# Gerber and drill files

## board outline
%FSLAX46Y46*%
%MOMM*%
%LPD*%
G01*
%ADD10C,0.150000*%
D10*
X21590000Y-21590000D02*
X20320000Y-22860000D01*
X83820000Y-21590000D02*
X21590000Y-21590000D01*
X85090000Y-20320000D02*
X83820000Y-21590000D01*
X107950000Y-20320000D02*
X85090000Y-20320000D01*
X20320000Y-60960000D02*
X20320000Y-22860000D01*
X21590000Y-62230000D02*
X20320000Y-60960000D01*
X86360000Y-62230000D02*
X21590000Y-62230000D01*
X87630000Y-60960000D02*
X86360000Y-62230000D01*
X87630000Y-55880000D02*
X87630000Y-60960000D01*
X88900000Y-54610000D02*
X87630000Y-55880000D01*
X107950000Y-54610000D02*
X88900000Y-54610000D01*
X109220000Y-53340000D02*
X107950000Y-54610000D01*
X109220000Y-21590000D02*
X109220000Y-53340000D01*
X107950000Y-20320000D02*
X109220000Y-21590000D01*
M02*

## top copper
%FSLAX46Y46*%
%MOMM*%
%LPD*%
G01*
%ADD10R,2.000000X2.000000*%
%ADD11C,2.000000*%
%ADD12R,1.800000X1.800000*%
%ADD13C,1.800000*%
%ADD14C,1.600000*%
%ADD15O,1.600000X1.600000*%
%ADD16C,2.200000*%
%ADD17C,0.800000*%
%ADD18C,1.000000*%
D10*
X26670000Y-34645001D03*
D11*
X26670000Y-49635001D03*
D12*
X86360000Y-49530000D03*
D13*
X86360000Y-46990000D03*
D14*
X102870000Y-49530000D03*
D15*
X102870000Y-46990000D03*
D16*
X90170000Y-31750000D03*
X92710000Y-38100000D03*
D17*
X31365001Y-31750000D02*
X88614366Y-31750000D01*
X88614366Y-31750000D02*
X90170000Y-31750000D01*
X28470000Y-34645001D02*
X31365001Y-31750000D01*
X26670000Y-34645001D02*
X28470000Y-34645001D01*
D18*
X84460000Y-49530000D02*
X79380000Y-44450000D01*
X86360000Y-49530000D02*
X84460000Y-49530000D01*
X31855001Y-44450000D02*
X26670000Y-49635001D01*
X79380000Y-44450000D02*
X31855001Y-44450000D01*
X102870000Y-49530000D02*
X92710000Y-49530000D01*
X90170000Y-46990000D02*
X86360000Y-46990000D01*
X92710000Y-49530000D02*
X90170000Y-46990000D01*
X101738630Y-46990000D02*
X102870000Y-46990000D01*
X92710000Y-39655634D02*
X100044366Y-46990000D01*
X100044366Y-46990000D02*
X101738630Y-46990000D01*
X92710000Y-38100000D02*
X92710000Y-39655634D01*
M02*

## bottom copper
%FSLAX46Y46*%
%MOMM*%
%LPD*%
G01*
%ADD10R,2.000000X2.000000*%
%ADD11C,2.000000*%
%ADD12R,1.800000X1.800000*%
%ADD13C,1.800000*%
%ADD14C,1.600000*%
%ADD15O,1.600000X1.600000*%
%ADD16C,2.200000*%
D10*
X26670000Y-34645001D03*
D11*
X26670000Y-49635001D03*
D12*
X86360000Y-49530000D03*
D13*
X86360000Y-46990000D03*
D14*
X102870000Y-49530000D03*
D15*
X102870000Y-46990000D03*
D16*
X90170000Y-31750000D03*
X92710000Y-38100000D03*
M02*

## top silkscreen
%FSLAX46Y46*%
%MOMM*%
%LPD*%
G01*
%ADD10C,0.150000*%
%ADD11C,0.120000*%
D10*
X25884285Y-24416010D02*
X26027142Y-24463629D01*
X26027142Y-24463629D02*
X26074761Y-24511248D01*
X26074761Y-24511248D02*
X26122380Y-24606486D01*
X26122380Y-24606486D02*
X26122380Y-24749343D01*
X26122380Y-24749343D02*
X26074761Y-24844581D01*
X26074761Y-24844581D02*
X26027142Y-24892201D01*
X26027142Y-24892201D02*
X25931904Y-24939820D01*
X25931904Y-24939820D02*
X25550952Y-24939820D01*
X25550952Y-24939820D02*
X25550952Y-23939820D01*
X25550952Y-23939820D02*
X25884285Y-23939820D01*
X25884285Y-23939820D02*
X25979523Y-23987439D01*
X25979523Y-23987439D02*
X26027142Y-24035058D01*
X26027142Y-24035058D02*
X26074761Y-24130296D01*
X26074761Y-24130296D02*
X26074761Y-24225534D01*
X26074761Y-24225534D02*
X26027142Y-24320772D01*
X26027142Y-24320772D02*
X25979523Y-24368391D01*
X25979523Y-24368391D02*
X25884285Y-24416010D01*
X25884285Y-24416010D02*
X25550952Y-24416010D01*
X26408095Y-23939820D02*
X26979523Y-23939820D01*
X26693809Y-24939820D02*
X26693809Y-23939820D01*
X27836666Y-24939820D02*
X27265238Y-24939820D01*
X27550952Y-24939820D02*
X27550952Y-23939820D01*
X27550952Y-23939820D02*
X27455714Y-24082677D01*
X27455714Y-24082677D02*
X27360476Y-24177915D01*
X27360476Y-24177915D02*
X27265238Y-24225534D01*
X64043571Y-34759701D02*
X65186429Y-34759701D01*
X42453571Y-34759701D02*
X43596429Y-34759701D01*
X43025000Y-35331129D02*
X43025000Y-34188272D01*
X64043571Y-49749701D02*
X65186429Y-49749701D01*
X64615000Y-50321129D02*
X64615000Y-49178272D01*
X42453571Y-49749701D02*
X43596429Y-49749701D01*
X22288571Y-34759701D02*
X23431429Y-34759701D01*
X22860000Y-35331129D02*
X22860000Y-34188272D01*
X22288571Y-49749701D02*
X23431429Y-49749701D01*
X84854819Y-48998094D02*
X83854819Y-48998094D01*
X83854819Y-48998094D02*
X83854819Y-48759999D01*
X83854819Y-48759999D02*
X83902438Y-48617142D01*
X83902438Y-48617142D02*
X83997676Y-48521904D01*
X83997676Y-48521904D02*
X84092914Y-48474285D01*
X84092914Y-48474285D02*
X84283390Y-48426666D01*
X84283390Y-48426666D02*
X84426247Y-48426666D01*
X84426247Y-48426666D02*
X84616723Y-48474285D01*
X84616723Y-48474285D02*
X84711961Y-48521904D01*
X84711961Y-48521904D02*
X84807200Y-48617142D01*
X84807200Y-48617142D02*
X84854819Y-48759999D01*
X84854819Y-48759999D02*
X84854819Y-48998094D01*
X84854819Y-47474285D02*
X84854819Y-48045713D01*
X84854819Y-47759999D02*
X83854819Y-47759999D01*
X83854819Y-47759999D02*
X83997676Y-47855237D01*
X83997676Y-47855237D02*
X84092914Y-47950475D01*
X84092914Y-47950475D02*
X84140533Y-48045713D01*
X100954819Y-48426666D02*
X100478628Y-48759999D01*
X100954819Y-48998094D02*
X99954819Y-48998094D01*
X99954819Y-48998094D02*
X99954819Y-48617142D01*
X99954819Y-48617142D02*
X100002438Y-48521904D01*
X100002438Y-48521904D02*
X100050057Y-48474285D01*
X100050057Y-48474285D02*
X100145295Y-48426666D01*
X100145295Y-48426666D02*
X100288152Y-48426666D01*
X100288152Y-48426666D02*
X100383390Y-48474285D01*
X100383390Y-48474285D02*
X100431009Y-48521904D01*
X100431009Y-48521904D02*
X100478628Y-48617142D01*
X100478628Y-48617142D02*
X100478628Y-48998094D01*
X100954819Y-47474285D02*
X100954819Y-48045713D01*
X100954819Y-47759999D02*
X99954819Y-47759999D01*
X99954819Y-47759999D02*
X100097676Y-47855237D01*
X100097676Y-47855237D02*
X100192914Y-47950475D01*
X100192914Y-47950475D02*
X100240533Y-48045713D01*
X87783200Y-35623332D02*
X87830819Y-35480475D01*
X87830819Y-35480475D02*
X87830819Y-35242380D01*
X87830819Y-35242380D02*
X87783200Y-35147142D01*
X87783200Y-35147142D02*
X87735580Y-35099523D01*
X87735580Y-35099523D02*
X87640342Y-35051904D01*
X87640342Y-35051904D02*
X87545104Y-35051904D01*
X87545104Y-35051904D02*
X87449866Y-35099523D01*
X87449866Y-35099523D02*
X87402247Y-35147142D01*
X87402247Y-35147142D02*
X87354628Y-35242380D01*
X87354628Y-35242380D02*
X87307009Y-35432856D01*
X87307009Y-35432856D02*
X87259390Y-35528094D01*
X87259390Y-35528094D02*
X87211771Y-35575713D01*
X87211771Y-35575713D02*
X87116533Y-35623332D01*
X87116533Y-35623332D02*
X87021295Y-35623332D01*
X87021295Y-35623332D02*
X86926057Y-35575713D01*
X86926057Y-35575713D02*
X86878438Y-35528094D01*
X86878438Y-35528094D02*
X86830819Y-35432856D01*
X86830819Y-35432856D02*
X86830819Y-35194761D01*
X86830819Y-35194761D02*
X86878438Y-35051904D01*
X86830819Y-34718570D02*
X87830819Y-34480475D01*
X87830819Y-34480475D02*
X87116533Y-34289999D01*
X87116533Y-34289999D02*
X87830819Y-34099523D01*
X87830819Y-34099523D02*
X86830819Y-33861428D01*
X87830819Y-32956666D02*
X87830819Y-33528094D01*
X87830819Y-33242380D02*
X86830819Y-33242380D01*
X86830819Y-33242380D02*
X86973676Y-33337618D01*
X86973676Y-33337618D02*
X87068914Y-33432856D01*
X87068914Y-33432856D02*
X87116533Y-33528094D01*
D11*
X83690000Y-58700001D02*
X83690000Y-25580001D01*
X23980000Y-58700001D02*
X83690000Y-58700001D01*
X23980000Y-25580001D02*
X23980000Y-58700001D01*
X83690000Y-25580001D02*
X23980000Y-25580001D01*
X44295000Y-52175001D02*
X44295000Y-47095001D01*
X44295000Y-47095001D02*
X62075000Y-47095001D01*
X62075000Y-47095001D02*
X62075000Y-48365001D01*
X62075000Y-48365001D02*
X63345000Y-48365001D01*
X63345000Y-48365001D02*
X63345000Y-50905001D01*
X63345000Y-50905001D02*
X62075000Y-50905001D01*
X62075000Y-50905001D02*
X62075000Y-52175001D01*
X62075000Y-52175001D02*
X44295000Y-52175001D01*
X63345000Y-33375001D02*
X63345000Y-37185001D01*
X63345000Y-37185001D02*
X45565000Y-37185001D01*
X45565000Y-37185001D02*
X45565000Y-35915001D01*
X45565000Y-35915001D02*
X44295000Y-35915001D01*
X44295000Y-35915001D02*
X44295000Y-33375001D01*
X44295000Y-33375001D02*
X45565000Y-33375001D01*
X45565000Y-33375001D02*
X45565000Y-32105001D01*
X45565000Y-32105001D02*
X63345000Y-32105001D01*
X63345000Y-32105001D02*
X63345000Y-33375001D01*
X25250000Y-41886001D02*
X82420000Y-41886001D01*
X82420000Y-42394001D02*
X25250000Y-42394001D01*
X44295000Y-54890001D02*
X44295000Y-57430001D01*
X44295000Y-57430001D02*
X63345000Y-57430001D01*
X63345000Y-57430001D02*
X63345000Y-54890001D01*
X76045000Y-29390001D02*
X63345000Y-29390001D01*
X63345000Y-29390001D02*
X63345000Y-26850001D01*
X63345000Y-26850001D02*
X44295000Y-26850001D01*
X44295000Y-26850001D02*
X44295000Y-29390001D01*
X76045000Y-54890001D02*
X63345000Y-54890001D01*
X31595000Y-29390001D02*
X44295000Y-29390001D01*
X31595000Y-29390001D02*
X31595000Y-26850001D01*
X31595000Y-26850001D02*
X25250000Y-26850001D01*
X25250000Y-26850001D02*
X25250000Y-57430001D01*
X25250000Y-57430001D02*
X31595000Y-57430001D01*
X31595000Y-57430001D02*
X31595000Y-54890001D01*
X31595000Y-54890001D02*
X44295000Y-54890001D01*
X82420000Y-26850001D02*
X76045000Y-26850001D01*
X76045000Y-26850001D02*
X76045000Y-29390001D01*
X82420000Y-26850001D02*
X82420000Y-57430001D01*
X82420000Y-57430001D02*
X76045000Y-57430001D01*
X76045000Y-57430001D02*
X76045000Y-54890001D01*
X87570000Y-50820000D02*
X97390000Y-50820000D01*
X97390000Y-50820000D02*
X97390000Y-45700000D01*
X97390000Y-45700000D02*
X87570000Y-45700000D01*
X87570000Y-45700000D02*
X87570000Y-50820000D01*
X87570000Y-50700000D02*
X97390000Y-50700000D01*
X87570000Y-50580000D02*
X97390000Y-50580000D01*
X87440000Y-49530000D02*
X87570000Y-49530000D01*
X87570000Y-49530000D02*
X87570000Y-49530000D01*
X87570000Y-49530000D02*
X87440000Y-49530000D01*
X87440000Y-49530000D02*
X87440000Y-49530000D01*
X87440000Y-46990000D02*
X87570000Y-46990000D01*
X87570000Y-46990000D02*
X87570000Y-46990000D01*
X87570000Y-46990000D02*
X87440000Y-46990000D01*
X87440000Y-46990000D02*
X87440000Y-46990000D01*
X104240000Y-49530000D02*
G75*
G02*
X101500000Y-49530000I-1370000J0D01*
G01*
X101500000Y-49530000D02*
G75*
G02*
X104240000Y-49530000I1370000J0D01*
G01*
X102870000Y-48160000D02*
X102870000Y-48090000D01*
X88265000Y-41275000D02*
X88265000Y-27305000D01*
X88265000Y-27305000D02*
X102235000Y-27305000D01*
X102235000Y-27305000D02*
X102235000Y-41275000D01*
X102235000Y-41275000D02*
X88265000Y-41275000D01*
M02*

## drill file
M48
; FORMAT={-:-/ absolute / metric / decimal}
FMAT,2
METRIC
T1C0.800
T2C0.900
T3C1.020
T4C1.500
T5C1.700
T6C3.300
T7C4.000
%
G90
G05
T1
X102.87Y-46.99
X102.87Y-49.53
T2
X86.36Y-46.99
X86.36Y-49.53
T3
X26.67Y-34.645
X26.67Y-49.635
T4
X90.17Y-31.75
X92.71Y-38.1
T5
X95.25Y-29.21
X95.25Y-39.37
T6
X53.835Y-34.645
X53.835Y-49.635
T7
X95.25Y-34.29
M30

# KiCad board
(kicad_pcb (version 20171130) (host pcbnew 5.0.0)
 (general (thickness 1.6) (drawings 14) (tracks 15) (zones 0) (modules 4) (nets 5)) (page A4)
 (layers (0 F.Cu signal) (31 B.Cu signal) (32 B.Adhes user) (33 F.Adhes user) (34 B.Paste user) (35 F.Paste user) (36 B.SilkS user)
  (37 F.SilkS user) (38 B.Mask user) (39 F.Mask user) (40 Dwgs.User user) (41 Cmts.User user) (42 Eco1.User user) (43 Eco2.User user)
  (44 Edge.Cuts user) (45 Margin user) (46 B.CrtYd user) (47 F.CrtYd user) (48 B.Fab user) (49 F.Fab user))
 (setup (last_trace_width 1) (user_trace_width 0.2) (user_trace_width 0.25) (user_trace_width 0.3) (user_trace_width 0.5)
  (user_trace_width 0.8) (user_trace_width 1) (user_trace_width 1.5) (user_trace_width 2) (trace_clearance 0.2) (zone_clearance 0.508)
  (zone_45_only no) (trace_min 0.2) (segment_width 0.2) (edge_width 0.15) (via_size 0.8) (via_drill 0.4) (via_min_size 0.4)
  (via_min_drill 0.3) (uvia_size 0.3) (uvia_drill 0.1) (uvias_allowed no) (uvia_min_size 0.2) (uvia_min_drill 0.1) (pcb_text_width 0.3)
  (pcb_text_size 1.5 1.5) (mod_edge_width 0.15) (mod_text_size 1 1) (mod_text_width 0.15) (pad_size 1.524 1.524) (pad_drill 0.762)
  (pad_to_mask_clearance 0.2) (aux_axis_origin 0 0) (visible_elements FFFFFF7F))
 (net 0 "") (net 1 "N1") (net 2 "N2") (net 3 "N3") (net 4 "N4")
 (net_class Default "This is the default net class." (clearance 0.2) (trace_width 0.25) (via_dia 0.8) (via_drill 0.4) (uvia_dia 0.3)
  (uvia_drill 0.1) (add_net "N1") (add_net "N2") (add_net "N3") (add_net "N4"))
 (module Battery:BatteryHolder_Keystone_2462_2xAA (layer F.Cu) (at 26.67 34.645001)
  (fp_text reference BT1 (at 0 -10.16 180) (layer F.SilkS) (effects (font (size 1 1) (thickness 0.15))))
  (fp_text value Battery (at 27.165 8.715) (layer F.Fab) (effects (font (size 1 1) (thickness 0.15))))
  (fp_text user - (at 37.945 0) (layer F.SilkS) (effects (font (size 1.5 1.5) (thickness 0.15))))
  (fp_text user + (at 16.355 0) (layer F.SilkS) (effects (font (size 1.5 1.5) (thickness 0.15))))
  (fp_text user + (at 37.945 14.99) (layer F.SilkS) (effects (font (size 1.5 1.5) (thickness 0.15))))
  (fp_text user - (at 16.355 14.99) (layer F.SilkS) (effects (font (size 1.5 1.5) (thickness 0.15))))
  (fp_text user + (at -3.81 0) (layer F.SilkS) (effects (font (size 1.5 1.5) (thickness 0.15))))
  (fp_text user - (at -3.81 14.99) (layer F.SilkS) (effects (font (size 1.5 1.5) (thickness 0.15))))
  (fp_line (start 57.02 24.055) (end 57.02 -9.065) (layer F.SilkS) (width 0.12))
  (fp_line (start -2.69 24.055) (end 57.02 24.055) (layer F.SilkS) (width 0.12))
  (fp_line (start -2.69 -9.065) (end -2.69 24.055) (layer F.SilkS) (width 0.12))
  (fp_line (start 57.02 -9.065) (end -2.69 -9.065) (layer F.SilkS) (width 0.12))
  (fp_line (start 17.625 17.53) (end 17.625 12.45) (layer F.SilkS) (width 0.12))
  (fp_line (start 17.625 12.45) (end 35.405 12.45) (layer F.SilkS) (width 0.12))
  (fp_line (start 35.405 12.45) (end 35.405 13.72) (layer F.SilkS) (width 0.12))
  (fp_line (start 35.405 13.72) (end 36.675 13.72) (layer F.SilkS) (width 0.12))
  (fp_line (start 36.675 13.72) (end 36.675 16.26) (layer F.SilkS) (width 0.12))
  (fp_line (start 36.675 16.26) (end 35.405 16.26) (layer F.SilkS) (width 0.12))
  (fp_line (start 35.405 16.26) (end 35.405 17.53) (layer F.SilkS) (width 0.12))
  (fp_line (start 35.405 17.53) (end 17.625 17.53) (layer F.SilkS) (width 0.12))
  (fp_line (start 36.675 -1.27) (end 36.675 2.54) (layer F.SilkS) (width 0.12))
  (fp_line (start 36.675 2.54) (end 18.895 2.54) (layer F.SilkS) (width 0.12))
  (fp_line (start 18.895 2.54) (end 18.895 1.27) (layer F.SilkS) (width 0.12))
  (fp_line (start 18.895 1.27) (end 17.625 1.27) (layer F.SilkS) (width 0.12))
  (fp_line (start 17.625 1.27) (end 17.625 -1.27) (layer F.SilkS) (width 0.12))
  (fp_line (start 17.625 -1.27) (end 18.895 -1.27) (layer F.SilkS) (width 0.12))
  (fp_line (start 18.895 -1.27) (end 18.895 -2.54) (layer F.SilkS) (width 0.12))
  (fp_line (start 18.895 -2.54) (end 36.675 -2.54) (layer F.SilkS) (width 0.12))
  (fp_line (start 36.675 -2.54) (end 36.675 -1.27) (layer F.SilkS) (width 0.12))
  (fp_line (start -1.42 7.241) (end 55.75 7.241) (layer F.SilkS) (width 0.12))
  (fp_line (start 55.75 7.749) (end -1.42 7.749) (layer F.SilkS) (width 0.12))
  (fp_line (start 17.625 20.245) (end 17.625 22.785) (layer F.SilkS) (width 0.12))
  (fp_line (start 17.625 22.785) (end 36.675 22.785) (layer F.SilkS) (width 0.12))
  (fp_line (start 36.675 22.785) (end 36.675 20.245) (layer F.SilkS) (width 0.12))
  (fp_line (start 49.375 -5.255) (end 36.675 -5.255) (layer F.SilkS) (width 0.12))
  (fp_line (start 36.675 -5.255) (end 36.675 -7.795) (layer F.SilkS) (width 0.12))
  (fp_line (start 36.675 -7.795) (end 17.625 -7.795) (layer F.SilkS) (width 0.12))
  (fp_line (start 17.625 -7.795) (end 17.625 -5.255) (layer F.SilkS) (width 0.12))
  (fp_line (start 49.375 20.245) (end 36.675 20.245) (layer F.SilkS) (width 0.12))
  (fp_line (start 4.925 -5.255) (end 17.625 -5.255) (layer F.SilkS) (width 0.12))
  (fp_line (start 4.925 -5.255) (end 4.925 -7.795) (layer F.SilkS) (width 0.12))
  (fp_line (start 4.925 -7.795) (end -1.42 -7.795) (layer F.SilkS) (width 0.12))
  (fp_line (start -1.42 -7.795) (end -1.42 22.785) (layer F.SilkS) (width 0.12))
  (fp_line (start -1.42 22.785) (end 4.925 22.785) (layer F.SilkS) (width 0.12))
  (fp_line (start 4.925 22.785) (end 4.925 20.245) (layer F.SilkS) (width 0.12))
  (fp_line (start 4.925 20.245) (end 17.625 20.245) (layer F.SilkS) (width 0.12))
  (fp_line (start 55.75 -7.795) (end 49.375 -7.795) (layer F.SilkS) (width 0.12))
  (fp_line (start 49.375 -7.795) (end 49.375 -5.255) (layer F.SilkS) (width 0.12))
  (fp_line (start 55.75 -7.795) (end 55.75 22.785) (layer F.SilkS) (width 0.12))
  (fp_line (start 55.75 22.785) (end 49.375 22.785) (layer F.SilkS) (width 0.12))
  (fp_line (start 49.375 22.785) (end 49.375 20.245) (layer F.SilkS) (width 0.12))
  (pad 1 thru_hole rect (at 0 0) (size 2 2) (drill 1.02) (layers *.Cu *.Mask) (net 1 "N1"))
  (pad 2 thru_hole circle (at 0 14.99) (size 2 2) (drill 1.02) (layers *.Cu *.Mask) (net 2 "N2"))
  (pad "" np_thru_hole circle (at 27.165 14.99) (size 3.3 3.3) (drill 3.3) (layers *.Cu *.Mask))
  (pad "" np_thru_hole circle (at 27.165 0) (size 3.3 3.3) (drill 3.3) (layers *.Cu *.Mask)))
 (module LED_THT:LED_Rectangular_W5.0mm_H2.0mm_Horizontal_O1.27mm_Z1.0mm (layer F.Cu) (at 86.36 49.53 90)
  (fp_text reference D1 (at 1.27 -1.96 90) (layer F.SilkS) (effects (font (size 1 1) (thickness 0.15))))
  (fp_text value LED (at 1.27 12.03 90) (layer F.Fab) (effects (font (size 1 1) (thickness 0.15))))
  (fp_line (start -1.29 1.21) (end -1.29 11.03) (layer F.SilkS) (width 0.12))
  (fp_line (start -1.29 11.03) (end 3.83 11.03) (layer F.SilkS) (width 0.12))
  (fp_line (start 3.83 11.03) (end 3.83 1.21) (layer F.SilkS) (width 0.12))
  (fp_line (start 3.83 1.21) (end -1.29 1.21) (layer F.SilkS) (width 0.12))
  (fp_line (start -1.17 1.21) (end -1.17 11.03) (layer F.SilkS) (width 0.12))
  (fp_line (start -1.05 1.21) (end -1.05 11.03) (layer F.SilkS) (width 0.12))
  (fp_line (start 0 1.08) (end 0 1.21) (layer F.SilkS) (width 0.12))
  (fp_line (start 0 1.21) (end 0 1.21) (layer F.SilkS) (width 0.12))
  (fp_line (start 0 1.21) (end 0 1.08) (layer F.SilkS) (width 0.12))
  (fp_line (start 0 1.08) (end 0 1.08) (layer F.SilkS) (width 0.12))
  (fp_line (start 2.54 1.08) (end 2.54 1.21) (layer F.SilkS) (width 0.12))
  (fp_line (start 2.54 1.21) (end 2.54 1.21) (layer F.SilkS) (width 0.12))
  (fp_line (start 2.54 1.21) (end 2.54 1.08) (layer F.SilkS) (width 0.12))
  (fp_line (start 2.54 1.08) (end 2.54 1.08) (layer F.SilkS) (width 0.12))
  (pad 1 thru_hole rect (at 0 0 90) (size 1.8 1.8) (drill 0.9) (layers *.Cu *.Mask) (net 2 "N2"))
  (pad 2 thru_hole circle (at 2.54 0 90) (size 1.8 1.8) (drill 0.9) (layers *.Cu *.Mask) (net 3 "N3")))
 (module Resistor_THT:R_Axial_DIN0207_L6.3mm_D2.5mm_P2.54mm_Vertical (layer F.Cu) (at 102.87 49.53 90)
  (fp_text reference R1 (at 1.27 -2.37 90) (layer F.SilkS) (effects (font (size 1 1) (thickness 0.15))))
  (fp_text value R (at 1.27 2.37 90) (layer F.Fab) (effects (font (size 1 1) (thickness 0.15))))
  (fp_circle (center 0 0) (end 1.37 0) (layer F.SilkS) (width 0.12))
  (fp_line (start 1.37 0) (end 1.44 0) (layer F.SilkS) (width 0.12))
  (pad 1 thru_hole circle (at 0 0 90) (size 1.6 1.6) (drill 0.8) (layers *.Cu *.Mask) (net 3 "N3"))
  (pad 2 thru_hole oval (at 2.54 0 90) (size 1.6 1.6) (drill 0.8) (layers *.Cu *.Mask) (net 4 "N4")))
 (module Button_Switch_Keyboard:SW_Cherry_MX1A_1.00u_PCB (layer F.Cu) (at 90.17 31.75 90)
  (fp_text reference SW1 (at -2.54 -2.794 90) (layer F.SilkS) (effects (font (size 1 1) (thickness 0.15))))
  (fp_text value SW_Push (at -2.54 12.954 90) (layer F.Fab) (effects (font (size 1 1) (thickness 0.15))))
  (fp_line (start -9.525 -1.905) (end 4.445 -1.905) (layer F.SilkS) (width 0.12))
  (fp_line (start 4.445 -1.905) (end 4.445 12.065) (layer F.SilkS) (width 0.12))
  (fp_line (start 4.445 12.065) (end -9.525 12.065) (layer F.SilkS) (width 0.12))
  (fp_line (start -9.525 12.065) (end -9.525 -1.905) (layer F.SilkS) (width 0.12))
  (pad 1 thru_hole circle (at 0 0 90) (size 2.2 2.2) (drill 1.5) (layers *.Cu *.Mask) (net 1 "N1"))
  (pad 2 thru_hole circle (at -6.35 2.54 90) (size 2.2 2.2) (drill 1.5) (layers *.Cu *.Mask) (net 4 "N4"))
  (pad "" np_thru_hole circle (at -2.54 5.08 90) (size 4 4) (drill 4) (layers *.Cu *.Mask))
  (pad "" np_thru_hole circle (at -7.62 5.08 90) (size 1.7 1.7) (drill 1.7) (layers *.Cu *.Mask))
  (pad "" np_thru_hole circle (at 2.54 5.08 90) (size 1.7 1.7) (drill 1.7) (layers *.Cu *.Mask)))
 (gr_line (start 21.59 21.59) (end 20.32 22.86) (layer Edge.Cuts) (width 0.15))
 (gr_line (start 83.82 21.59) (end 21.59 21.59) (layer Edge.Cuts) (width 0.15))
 (gr_line (start 85.09 20.32) (end 83.82 21.59) (layer Edge.Cuts) (width 0.15))
 (gr_line (start 107.95 20.32) (end 85.09 20.32) (layer Edge.Cuts) (width 0.15))
 (gr_line (start 20.32 60.96) (end 20.32 22.86) (layer Edge.Cuts) (width 0.15))
 (gr_line (start 21.59 62.23) (end 20.32 60.96) (layer Edge.Cuts) (width 0.15))
 (gr_line (start 86.36 62.23) (end 21.59 62.23) (layer Edge.Cuts) (width 0.15))
 (gr_line (start 87.63 60.96) (end 86.36 62.23) (layer Edge.Cuts) (width 0.15))
 (gr_line (start 87.63 55.88) (end 87.63 60.96) (layer Edge.Cuts) (width 0.15))
 (gr_line (start 88.9 54.61) (end 87.63 55.88) (layer Edge.Cuts) (width 0.15))
 (gr_line (start 107.95 54.61) (end 88.9 54.61) (layer Edge.Cuts) (width 0.15))
 (gr_line (start 109.22 53.34) (end 107.95 54.61) (layer Edge.Cuts) (width 0.15))
 (gr_line (start 109.22 21.59) (end 109.22 53.34) (layer Edge.Cuts) (width 0.15))
 (gr_line (start 107.95 20.32) (end 109.22 21.59) (layer Edge.Cuts) (width 0.15))
 (segment (start 31.365001 31.75) (end 88.614366 31.75) (width 0.8) (layer F.Cu) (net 1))
 (segment (start 88.614366 31.75) (end 90.17 31.75) (width 0.8) (layer F.Cu) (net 1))
 (segment (start 28.47 34.645001) (end 31.365001 31.75) (width 0.8) (layer F.Cu) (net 1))
 (segment (start 26.67 34.645001) (end 28.47 34.645001) (width 0.8) (layer F.Cu) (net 1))
 (segment (start 84.46 49.53) (end 79.38 44.45) (width 1) (layer F.Cu) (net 2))
 (segment (start 86.36 49.53) (end 84.46 49.53) (width 1) (layer F.Cu) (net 2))
 (segment (start 31.855001 44.45) (end 26.67 49.635001) (width 1) (layer F.Cu) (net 2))
 (segment (start 79.38 44.45) (end 31.855001 44.45) (width 1) (layer F.Cu) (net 2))
 (segment (start 102.87 49.53) (end 92.71 49.53) (width 1) (layer F.Cu) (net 3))
 (segment (start 90.17 46.99) (end 86.36 46.99) (width 1) (layer F.Cu) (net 3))
 (segment (start 92.71 49.53) (end 90.17 46.99) (width 1) (layer F.Cu) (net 3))
 (segment (start 101.73863 46.99) (end 102.87 46.99) (width 1) (layer F.Cu) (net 4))
 (segment (start 92.71 39.655634) (end 100.044366 46.99) (width 1) (layer F.Cu) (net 4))
 (segment (start 100.044366 46.99) (end 101.73863 46.99) (width 1) (layer F.Cu) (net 4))
 (segment (start 92.71 38.1) (end 92.71 39.655634) (width 1) (layer F.Cu) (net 4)))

